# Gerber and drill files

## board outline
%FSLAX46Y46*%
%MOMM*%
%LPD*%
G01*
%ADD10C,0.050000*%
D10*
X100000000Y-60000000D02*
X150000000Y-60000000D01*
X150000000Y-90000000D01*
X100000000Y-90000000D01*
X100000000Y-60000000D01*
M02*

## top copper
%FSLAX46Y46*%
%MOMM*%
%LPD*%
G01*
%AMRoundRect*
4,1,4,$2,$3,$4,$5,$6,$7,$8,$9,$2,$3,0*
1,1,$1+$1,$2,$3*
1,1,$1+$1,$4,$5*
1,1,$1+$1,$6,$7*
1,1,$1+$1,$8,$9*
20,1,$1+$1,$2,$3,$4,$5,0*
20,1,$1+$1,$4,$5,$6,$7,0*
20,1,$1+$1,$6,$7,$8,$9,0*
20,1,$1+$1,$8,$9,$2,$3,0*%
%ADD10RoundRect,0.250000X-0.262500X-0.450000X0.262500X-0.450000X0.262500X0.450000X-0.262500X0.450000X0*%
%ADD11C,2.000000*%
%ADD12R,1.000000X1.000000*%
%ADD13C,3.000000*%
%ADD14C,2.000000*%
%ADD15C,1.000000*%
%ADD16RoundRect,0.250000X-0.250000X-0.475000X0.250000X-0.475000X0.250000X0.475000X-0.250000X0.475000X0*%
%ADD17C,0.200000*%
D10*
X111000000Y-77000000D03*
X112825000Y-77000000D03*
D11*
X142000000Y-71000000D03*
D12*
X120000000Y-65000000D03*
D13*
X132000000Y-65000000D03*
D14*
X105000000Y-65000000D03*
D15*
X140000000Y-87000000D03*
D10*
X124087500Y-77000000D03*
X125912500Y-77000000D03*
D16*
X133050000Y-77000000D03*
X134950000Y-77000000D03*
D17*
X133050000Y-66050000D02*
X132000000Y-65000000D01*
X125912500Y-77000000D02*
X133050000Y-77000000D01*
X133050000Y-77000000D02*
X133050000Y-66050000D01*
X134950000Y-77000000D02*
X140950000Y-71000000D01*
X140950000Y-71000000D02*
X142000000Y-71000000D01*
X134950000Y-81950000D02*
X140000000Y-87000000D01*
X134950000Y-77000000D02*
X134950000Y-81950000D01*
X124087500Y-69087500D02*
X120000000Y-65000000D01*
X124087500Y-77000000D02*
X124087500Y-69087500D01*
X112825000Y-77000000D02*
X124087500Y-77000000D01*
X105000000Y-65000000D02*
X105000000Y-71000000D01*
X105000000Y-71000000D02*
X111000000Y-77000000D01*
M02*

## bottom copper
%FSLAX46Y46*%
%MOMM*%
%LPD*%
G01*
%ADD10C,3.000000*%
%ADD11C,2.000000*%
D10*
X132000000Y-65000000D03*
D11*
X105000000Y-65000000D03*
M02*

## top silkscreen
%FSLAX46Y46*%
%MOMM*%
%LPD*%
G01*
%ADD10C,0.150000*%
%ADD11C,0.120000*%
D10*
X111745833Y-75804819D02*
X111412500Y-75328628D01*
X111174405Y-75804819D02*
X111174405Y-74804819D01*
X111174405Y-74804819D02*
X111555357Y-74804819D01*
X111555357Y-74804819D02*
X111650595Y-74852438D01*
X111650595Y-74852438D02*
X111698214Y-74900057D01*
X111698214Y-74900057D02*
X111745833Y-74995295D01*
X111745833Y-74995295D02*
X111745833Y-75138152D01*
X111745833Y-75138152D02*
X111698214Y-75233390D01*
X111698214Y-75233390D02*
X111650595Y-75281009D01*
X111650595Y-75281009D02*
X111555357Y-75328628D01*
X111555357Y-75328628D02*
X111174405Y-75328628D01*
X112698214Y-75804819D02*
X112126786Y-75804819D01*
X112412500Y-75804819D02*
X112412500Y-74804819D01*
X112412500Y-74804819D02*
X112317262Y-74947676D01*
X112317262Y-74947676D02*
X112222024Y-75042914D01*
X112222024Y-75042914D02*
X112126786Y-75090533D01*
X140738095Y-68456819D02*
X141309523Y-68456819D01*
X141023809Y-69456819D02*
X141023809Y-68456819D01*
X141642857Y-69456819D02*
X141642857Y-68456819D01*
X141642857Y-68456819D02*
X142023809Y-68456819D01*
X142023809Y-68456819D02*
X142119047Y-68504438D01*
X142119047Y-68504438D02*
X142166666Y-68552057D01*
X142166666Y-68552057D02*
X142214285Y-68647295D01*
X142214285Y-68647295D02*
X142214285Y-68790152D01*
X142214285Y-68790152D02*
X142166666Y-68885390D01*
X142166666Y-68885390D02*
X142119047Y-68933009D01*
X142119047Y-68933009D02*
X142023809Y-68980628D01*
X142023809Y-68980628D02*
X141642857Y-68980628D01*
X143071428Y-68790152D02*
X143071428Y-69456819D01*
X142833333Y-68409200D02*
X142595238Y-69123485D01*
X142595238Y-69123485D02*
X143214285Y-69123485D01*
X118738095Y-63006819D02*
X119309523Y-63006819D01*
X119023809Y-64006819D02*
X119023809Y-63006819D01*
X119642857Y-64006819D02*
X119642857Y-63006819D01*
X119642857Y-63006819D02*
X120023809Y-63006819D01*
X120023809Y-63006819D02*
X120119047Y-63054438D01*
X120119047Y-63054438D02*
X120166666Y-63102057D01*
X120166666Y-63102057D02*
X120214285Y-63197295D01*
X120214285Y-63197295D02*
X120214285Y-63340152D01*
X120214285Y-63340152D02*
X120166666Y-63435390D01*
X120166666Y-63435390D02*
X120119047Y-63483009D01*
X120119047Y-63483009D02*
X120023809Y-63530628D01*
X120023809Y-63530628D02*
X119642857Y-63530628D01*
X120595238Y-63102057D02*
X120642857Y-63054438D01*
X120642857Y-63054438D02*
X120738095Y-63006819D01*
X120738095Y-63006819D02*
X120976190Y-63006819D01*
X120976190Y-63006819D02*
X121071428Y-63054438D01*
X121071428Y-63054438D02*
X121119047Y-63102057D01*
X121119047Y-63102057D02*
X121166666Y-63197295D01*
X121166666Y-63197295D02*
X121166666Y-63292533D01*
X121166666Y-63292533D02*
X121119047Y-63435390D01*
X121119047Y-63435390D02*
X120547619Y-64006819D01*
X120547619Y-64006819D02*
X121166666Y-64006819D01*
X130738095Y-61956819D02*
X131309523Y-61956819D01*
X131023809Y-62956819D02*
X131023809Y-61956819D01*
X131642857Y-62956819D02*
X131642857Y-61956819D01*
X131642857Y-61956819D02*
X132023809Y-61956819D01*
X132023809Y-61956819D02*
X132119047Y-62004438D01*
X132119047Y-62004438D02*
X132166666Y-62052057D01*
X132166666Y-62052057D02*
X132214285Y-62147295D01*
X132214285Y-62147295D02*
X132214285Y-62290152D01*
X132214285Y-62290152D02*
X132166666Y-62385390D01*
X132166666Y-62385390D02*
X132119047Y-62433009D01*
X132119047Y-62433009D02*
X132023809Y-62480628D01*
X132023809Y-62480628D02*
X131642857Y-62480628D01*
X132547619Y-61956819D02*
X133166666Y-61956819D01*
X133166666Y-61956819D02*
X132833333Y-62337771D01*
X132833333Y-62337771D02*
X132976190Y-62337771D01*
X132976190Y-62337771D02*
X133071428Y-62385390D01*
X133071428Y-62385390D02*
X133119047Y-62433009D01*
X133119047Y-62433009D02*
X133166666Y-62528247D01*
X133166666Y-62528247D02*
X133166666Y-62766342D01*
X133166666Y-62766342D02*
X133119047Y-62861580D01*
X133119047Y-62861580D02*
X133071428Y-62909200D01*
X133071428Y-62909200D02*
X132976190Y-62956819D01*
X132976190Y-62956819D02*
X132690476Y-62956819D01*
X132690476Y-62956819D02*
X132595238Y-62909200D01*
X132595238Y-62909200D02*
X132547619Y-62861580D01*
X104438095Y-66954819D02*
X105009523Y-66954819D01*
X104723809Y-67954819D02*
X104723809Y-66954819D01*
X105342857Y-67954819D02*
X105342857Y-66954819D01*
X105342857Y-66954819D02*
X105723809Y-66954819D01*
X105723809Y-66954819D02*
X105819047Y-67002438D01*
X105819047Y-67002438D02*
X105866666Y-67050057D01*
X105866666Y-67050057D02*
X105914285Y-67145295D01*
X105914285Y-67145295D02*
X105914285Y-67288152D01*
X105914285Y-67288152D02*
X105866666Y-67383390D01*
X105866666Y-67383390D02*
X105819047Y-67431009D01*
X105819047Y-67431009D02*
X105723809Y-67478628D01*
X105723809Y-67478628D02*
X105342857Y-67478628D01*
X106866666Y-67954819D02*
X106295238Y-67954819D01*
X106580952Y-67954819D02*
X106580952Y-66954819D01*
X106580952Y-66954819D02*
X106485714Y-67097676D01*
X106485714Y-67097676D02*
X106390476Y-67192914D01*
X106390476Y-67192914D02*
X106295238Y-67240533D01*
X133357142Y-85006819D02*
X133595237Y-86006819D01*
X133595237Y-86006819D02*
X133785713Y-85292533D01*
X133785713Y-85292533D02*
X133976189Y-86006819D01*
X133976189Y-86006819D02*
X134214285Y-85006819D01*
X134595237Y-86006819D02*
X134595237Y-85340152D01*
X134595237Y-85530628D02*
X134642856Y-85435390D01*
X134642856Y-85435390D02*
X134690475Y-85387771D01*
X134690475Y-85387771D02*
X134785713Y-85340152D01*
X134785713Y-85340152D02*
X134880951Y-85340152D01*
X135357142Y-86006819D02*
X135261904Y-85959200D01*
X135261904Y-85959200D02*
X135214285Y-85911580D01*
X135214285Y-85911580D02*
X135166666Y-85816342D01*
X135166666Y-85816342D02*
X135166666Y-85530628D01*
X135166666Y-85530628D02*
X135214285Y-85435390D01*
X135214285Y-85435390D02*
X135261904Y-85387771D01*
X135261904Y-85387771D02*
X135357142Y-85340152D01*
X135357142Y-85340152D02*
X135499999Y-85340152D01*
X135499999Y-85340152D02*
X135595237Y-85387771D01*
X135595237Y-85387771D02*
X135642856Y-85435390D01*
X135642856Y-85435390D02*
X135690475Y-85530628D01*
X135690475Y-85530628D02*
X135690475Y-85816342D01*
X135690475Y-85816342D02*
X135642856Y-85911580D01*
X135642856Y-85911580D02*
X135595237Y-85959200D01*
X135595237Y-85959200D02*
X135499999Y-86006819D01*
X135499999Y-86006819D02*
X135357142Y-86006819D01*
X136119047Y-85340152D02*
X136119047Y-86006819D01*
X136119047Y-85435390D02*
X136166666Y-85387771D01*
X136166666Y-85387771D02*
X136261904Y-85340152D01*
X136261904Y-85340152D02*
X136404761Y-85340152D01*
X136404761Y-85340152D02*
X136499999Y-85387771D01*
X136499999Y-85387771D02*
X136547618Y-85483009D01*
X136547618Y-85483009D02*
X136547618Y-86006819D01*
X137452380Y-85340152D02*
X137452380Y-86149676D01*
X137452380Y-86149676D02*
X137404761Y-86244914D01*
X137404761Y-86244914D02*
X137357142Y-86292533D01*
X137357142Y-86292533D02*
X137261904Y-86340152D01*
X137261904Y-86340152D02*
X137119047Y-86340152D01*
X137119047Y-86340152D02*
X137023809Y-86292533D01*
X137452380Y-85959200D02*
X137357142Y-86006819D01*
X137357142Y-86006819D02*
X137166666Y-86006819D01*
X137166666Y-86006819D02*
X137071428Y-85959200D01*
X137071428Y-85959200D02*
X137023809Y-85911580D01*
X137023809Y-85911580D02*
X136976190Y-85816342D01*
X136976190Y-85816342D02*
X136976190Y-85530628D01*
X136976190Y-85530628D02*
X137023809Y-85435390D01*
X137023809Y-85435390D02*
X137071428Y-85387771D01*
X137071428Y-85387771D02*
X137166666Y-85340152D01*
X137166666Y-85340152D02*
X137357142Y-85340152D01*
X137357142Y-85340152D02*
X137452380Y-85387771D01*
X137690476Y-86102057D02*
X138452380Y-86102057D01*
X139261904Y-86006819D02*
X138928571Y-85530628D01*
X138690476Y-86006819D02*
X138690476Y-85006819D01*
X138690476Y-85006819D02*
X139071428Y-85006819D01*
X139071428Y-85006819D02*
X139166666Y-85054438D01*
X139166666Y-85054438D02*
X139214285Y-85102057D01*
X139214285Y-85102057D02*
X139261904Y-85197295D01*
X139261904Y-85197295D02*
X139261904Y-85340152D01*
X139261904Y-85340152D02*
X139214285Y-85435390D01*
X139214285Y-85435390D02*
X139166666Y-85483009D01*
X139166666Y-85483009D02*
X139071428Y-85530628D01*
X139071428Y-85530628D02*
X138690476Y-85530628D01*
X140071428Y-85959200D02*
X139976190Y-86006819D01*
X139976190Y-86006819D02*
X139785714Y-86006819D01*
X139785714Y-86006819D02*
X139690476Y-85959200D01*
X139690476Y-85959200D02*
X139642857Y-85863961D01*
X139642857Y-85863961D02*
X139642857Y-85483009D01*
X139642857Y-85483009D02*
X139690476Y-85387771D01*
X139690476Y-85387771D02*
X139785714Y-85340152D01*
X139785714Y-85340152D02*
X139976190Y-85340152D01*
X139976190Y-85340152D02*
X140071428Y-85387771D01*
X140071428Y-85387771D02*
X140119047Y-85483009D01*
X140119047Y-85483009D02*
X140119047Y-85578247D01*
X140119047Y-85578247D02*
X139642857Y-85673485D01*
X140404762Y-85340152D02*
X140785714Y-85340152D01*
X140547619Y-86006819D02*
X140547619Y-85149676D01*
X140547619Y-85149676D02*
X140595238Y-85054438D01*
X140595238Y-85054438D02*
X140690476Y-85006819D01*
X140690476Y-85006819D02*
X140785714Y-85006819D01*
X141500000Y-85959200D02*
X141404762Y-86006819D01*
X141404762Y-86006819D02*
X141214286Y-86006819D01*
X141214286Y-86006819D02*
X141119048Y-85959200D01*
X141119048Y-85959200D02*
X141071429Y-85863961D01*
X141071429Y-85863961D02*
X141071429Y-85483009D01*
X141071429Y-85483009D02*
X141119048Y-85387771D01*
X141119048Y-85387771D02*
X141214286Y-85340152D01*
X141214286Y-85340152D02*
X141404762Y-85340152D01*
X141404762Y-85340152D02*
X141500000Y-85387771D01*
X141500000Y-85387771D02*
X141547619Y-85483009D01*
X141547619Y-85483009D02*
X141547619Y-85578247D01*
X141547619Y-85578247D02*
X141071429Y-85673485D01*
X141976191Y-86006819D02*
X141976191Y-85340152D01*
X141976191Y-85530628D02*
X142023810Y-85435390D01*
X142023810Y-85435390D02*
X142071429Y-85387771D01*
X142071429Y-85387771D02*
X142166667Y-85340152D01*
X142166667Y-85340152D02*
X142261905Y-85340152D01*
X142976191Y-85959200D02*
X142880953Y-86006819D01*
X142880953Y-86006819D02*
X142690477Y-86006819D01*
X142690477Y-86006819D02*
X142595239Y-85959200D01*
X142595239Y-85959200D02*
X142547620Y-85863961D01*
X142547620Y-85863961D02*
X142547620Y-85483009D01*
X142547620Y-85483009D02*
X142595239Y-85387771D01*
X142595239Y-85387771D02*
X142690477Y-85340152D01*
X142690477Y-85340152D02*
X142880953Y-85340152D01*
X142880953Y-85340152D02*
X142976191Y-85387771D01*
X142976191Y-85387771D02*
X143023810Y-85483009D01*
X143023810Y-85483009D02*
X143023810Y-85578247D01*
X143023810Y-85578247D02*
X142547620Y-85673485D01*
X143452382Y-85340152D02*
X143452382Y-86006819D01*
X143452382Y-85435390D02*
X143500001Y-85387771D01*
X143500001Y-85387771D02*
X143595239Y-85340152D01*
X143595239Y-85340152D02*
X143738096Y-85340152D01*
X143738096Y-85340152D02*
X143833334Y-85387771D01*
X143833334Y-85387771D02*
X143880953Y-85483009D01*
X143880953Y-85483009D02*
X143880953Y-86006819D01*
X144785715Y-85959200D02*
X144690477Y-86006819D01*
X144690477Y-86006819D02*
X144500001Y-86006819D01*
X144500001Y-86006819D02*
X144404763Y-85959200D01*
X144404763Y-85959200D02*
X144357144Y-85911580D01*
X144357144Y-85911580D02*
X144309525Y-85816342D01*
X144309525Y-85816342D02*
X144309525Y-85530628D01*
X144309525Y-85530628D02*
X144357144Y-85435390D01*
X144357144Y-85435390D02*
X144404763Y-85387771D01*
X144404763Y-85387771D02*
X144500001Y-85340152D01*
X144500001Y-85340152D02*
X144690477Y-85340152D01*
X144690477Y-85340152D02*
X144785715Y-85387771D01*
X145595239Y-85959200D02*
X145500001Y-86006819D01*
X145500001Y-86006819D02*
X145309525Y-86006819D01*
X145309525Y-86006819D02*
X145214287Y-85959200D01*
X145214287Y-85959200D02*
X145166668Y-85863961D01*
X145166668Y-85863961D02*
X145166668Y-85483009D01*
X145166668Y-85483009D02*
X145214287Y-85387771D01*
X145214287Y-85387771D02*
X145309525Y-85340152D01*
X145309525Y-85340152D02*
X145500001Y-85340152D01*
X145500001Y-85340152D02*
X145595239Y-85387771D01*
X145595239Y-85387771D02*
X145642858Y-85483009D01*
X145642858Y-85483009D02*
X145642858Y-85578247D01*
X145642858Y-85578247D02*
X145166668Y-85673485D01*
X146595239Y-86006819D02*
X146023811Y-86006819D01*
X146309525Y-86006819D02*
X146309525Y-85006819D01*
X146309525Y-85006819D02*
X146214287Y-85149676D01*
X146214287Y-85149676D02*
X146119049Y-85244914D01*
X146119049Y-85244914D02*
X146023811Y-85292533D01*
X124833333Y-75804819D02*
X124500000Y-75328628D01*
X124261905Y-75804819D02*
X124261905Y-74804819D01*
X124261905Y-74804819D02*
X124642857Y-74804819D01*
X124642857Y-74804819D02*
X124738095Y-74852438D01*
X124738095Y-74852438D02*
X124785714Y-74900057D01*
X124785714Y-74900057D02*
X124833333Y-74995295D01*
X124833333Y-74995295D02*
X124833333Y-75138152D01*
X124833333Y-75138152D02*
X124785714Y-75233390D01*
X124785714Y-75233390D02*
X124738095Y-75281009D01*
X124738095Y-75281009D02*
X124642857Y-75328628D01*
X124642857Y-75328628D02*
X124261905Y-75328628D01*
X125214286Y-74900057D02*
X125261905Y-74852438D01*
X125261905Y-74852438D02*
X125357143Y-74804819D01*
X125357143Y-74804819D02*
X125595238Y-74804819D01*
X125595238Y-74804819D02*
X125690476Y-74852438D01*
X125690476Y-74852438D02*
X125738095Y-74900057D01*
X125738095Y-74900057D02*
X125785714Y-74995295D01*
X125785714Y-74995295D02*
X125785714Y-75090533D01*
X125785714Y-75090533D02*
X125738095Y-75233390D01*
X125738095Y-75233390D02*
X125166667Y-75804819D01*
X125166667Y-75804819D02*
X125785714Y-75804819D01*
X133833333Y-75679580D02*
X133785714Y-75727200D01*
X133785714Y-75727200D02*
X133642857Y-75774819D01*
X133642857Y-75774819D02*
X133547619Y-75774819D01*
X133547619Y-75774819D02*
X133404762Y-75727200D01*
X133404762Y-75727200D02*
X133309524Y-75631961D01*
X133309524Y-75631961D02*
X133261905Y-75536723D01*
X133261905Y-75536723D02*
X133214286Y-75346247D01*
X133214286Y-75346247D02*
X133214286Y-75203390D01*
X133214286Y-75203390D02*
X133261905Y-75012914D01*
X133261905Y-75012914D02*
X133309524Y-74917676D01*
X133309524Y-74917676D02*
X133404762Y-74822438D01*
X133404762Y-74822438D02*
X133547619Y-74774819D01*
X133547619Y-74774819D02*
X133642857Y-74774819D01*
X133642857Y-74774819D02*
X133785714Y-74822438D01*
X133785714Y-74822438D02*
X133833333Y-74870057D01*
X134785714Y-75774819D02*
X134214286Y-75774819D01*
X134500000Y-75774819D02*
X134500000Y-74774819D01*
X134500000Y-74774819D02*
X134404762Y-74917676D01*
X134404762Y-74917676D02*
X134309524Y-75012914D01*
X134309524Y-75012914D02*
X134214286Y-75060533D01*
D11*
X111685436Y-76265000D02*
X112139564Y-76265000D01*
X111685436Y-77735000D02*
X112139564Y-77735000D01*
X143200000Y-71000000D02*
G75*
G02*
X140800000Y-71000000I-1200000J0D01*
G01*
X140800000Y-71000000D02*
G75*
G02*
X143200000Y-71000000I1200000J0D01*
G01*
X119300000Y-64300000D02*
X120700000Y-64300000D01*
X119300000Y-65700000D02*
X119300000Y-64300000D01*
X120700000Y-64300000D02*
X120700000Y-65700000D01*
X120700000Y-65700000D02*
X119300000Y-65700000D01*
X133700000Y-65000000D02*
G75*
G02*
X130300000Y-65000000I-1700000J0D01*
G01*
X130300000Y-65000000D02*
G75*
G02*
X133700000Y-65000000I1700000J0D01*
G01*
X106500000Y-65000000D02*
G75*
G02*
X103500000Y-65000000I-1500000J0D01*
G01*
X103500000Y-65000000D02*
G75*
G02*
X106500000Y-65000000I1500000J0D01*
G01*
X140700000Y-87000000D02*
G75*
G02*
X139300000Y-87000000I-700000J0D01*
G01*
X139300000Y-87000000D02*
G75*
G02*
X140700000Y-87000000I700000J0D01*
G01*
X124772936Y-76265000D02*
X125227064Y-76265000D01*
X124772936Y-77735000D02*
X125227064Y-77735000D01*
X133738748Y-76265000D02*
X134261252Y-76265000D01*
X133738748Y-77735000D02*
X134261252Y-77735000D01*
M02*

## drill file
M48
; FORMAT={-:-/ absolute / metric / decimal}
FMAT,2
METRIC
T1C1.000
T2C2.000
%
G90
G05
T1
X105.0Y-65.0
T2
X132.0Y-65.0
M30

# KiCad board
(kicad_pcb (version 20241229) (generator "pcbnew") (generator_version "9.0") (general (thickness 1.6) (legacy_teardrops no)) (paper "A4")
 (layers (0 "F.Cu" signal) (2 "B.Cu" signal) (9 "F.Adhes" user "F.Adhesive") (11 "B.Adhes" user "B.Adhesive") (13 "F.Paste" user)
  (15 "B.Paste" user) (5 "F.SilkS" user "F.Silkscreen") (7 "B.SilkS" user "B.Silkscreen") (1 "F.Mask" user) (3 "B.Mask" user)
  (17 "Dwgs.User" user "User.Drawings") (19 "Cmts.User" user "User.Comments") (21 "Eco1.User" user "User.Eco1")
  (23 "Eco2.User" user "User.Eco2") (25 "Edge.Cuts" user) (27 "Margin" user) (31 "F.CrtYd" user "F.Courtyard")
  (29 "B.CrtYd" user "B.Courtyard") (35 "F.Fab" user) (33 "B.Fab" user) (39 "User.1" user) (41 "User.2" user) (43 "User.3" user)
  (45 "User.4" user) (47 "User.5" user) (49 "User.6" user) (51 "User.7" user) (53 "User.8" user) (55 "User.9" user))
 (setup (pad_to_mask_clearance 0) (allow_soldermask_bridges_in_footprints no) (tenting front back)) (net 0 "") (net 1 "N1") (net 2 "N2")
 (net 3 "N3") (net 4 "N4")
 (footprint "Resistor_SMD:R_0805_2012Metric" (layer "F.Cu") (at 111.9125 77)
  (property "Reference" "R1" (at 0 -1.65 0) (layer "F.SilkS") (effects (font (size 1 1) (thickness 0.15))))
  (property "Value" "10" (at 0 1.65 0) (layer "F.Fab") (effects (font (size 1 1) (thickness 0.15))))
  (fp_line (start -0.227064 -0.735) (end 0.227064 -0.735) (stroke (width 0.12) (type solid)) (layer "F.SilkS"))
  (fp_line (start -0.227064 0.735) (end 0.227064 0.735) (stroke (width 0.12) (type solid)) (layer "F.SilkS"))
  (pad "1" smd roundrect (at -0.9125 0) (size 1.025 1.4) (layers "F.Cu" "F.Mask" "F.Paste") (roundrect_rratio 0.243902) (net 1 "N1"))
  (pad "2" smd roundrect (at 0.9125 0) (size 1.025 1.4) (layers "F.Cu" "F.Mask" "F.Paste") (roundrect_rratio 0.243902) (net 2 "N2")))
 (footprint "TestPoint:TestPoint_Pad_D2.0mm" (layer "F.Cu") (at 142 71)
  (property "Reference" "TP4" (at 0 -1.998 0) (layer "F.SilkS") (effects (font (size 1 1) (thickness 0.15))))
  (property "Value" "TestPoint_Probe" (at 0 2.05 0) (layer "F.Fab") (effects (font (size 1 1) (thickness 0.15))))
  (fp_circle (center 0 0) (end 0 1.2) (stroke (width 0.12) (type solid)) (fill no) (layer "F.SilkS"))
  (pad "1" smd circle (at 0 0) (size 2 2) (layers "F.Cu" "F.Mask") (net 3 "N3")))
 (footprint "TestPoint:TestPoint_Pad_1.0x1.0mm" (layer "F.Cu") (at 120 65)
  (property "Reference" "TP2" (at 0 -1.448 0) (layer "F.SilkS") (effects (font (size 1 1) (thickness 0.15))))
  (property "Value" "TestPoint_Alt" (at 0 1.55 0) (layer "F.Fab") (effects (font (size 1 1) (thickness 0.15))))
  (fp_line (start -0.7 -0.7) (end 0.7 -0.7) (stroke (width 0.12) (type solid)) (layer "F.SilkS"))
  (fp_line (start -0.7 0.7) (end -0.7 -0.7) (stroke (width 0.12) (type solid)) (layer "F.SilkS"))
  (fp_line (start 0.7 -0.7) (end 0.7 0.7) (stroke (width 0.12) (type solid)) (layer "F.SilkS"))
  (fp_line (start 0.7 0.7) (end -0.7 0.7) (stroke (width 0.12) (type solid)) (layer "F.SilkS"))
  (pad "1" smd rect (at 0 0) (size 1 1) (layers "F.Cu" "F.Mask") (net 2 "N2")))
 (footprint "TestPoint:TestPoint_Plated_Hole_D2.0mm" (layer "F.Cu") (at 132 65)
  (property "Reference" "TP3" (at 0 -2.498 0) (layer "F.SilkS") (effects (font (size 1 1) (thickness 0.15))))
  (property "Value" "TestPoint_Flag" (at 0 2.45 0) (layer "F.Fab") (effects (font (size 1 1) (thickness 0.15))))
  (fp_circle (center 0 0) (end 0 -1.7) (stroke (width 0.12) (type solid)) (fill no) (layer "F.SilkS"))
  (pad "1" thru_hole circle (at 0 0) (size 3 3) (drill 2) (layers "*.Cu" "*.Mask") (remove_unused_layers no) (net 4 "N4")))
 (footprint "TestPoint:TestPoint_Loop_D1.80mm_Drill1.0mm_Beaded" (layer "F.Cu") (at 105 65)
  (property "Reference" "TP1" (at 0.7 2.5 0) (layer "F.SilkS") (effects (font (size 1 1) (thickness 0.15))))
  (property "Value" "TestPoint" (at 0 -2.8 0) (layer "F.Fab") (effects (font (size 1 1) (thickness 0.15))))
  (fp_circle (center 0 0) (end 1.5 0) (stroke (width 0.12) (type solid)) (fill no) (layer "F.SilkS"))
  (pad "1" thru_hole circle (at 0 0) (size 2 2) (drill 1) (layers "*.Cu" "*.Mask") (remove_unused_layers no) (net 1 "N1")))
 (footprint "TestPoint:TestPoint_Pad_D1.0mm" (layer "F.Cu") (at 140 87)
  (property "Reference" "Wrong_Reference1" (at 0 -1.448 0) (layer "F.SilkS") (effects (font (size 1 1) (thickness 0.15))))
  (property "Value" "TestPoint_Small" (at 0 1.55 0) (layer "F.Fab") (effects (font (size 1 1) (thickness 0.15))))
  (fp_circle (center 0 0) (end 0 0.7) (stroke (width 0.12) (type solid)) (fill no) (layer "F.SilkS"))
  (pad "1" smd circle (at 0 0) (size 1 1) (layers "F.Cu" "F.Mask") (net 3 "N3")))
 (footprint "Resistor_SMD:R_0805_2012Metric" (layer "F.Cu") (at 125 77)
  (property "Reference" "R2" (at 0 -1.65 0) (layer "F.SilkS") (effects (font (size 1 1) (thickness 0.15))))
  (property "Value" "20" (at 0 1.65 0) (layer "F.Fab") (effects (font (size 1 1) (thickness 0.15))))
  (fp_line (start -0.227064 -0.735) (end 0.227064 -0.735) (stroke (width 0.12) (type solid)) (layer "F.SilkS"))
  (fp_line (start -0.227064 0.735) (end 0.227064 0.735) (stroke (width 0.12) (type solid)) (layer "F.SilkS"))
  (pad "1" smd roundrect (at -0.9125 0) (size 1.025 1.4) (layers "F.Cu" "F.Mask" "F.Paste") (roundrect_rratio 0.243902) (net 2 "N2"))
  (pad "2" smd roundrect (at 0.9125 0) (size 1.025 1.4) (layers "F.Cu" "F.Mask" "F.Paste") (roundrect_rratio 0.243902) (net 4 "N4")))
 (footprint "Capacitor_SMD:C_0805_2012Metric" (layer "F.Cu") (at 134 77)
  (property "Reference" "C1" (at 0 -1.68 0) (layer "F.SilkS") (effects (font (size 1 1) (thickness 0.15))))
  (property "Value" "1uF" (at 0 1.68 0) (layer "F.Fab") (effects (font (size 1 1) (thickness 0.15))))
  (fp_line (start -0.261252 -0.735) (end 0.261252 -0.735) (stroke (width 0.12) (type solid)) (layer "F.SilkS"))
  (fp_line (start -0.261252 0.735) (end 0.261252 0.735) (stroke (width 0.12) (type solid)) (layer "F.SilkS"))
  (pad "1" smd roundrect (at -0.95 0) (size 1 1.45) (layers "F.Cu" "F.Mask" "F.Paste") (roundrect_rratio 0.25) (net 4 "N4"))
  (pad "2" smd roundrect (at 0.95 0) (size 1 1.45) (layers "F.Cu" "F.Mask" "F.Paste") (roundrect_rratio 0.25) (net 3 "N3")))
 (gr_rect (start 100 60) (end 150 90) (stroke (width 0.05) (type default)) (fill no) (layer "Edge.Cuts"))
 (segment (start 133.05 66.05) (end 132 65) (width 0.2) (layer "F.Cu") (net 4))
 (segment (start 125.9125 77) (end 133.05 77) (width 0.2) (layer "F.Cu") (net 4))
 (segment (start 133.05 77) (end 133.05 66.05) (width 0.2) (layer "F.Cu") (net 4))
 (segment (start 134.95 77) (end 140.95 71) (width 0.2) (layer "F.Cu") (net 3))
 (segment (start 140.95 71) (end 142 71) (width 0.2) (layer "F.Cu") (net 3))
 (segment (start 134.95 81.95) (end 140 87) (width 0.2) (layer "F.Cu") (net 3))
 (segment (start 134.95 77) (end 134.95 81.95) (width 0.2) (layer "F.Cu") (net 3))
 (segment (start 124.0875 69.0875) (end 120 65) (width 0.2) (layer "F.Cu") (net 2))
 (segment (start 124.0875 77) (end 124.0875 69.0875) (width 0.2) (layer "F.Cu") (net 2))
 (segment (start 112.825 77) (end 124.0875 77) (width 0.2) (layer "F.Cu") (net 2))
 (segment (start 105 65) (end 105 71) (width 0.2) (layer "F.Cu") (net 1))
 (segment (start 105 71) (end 111 77) (width 0.2) (layer "F.Cu") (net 1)))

